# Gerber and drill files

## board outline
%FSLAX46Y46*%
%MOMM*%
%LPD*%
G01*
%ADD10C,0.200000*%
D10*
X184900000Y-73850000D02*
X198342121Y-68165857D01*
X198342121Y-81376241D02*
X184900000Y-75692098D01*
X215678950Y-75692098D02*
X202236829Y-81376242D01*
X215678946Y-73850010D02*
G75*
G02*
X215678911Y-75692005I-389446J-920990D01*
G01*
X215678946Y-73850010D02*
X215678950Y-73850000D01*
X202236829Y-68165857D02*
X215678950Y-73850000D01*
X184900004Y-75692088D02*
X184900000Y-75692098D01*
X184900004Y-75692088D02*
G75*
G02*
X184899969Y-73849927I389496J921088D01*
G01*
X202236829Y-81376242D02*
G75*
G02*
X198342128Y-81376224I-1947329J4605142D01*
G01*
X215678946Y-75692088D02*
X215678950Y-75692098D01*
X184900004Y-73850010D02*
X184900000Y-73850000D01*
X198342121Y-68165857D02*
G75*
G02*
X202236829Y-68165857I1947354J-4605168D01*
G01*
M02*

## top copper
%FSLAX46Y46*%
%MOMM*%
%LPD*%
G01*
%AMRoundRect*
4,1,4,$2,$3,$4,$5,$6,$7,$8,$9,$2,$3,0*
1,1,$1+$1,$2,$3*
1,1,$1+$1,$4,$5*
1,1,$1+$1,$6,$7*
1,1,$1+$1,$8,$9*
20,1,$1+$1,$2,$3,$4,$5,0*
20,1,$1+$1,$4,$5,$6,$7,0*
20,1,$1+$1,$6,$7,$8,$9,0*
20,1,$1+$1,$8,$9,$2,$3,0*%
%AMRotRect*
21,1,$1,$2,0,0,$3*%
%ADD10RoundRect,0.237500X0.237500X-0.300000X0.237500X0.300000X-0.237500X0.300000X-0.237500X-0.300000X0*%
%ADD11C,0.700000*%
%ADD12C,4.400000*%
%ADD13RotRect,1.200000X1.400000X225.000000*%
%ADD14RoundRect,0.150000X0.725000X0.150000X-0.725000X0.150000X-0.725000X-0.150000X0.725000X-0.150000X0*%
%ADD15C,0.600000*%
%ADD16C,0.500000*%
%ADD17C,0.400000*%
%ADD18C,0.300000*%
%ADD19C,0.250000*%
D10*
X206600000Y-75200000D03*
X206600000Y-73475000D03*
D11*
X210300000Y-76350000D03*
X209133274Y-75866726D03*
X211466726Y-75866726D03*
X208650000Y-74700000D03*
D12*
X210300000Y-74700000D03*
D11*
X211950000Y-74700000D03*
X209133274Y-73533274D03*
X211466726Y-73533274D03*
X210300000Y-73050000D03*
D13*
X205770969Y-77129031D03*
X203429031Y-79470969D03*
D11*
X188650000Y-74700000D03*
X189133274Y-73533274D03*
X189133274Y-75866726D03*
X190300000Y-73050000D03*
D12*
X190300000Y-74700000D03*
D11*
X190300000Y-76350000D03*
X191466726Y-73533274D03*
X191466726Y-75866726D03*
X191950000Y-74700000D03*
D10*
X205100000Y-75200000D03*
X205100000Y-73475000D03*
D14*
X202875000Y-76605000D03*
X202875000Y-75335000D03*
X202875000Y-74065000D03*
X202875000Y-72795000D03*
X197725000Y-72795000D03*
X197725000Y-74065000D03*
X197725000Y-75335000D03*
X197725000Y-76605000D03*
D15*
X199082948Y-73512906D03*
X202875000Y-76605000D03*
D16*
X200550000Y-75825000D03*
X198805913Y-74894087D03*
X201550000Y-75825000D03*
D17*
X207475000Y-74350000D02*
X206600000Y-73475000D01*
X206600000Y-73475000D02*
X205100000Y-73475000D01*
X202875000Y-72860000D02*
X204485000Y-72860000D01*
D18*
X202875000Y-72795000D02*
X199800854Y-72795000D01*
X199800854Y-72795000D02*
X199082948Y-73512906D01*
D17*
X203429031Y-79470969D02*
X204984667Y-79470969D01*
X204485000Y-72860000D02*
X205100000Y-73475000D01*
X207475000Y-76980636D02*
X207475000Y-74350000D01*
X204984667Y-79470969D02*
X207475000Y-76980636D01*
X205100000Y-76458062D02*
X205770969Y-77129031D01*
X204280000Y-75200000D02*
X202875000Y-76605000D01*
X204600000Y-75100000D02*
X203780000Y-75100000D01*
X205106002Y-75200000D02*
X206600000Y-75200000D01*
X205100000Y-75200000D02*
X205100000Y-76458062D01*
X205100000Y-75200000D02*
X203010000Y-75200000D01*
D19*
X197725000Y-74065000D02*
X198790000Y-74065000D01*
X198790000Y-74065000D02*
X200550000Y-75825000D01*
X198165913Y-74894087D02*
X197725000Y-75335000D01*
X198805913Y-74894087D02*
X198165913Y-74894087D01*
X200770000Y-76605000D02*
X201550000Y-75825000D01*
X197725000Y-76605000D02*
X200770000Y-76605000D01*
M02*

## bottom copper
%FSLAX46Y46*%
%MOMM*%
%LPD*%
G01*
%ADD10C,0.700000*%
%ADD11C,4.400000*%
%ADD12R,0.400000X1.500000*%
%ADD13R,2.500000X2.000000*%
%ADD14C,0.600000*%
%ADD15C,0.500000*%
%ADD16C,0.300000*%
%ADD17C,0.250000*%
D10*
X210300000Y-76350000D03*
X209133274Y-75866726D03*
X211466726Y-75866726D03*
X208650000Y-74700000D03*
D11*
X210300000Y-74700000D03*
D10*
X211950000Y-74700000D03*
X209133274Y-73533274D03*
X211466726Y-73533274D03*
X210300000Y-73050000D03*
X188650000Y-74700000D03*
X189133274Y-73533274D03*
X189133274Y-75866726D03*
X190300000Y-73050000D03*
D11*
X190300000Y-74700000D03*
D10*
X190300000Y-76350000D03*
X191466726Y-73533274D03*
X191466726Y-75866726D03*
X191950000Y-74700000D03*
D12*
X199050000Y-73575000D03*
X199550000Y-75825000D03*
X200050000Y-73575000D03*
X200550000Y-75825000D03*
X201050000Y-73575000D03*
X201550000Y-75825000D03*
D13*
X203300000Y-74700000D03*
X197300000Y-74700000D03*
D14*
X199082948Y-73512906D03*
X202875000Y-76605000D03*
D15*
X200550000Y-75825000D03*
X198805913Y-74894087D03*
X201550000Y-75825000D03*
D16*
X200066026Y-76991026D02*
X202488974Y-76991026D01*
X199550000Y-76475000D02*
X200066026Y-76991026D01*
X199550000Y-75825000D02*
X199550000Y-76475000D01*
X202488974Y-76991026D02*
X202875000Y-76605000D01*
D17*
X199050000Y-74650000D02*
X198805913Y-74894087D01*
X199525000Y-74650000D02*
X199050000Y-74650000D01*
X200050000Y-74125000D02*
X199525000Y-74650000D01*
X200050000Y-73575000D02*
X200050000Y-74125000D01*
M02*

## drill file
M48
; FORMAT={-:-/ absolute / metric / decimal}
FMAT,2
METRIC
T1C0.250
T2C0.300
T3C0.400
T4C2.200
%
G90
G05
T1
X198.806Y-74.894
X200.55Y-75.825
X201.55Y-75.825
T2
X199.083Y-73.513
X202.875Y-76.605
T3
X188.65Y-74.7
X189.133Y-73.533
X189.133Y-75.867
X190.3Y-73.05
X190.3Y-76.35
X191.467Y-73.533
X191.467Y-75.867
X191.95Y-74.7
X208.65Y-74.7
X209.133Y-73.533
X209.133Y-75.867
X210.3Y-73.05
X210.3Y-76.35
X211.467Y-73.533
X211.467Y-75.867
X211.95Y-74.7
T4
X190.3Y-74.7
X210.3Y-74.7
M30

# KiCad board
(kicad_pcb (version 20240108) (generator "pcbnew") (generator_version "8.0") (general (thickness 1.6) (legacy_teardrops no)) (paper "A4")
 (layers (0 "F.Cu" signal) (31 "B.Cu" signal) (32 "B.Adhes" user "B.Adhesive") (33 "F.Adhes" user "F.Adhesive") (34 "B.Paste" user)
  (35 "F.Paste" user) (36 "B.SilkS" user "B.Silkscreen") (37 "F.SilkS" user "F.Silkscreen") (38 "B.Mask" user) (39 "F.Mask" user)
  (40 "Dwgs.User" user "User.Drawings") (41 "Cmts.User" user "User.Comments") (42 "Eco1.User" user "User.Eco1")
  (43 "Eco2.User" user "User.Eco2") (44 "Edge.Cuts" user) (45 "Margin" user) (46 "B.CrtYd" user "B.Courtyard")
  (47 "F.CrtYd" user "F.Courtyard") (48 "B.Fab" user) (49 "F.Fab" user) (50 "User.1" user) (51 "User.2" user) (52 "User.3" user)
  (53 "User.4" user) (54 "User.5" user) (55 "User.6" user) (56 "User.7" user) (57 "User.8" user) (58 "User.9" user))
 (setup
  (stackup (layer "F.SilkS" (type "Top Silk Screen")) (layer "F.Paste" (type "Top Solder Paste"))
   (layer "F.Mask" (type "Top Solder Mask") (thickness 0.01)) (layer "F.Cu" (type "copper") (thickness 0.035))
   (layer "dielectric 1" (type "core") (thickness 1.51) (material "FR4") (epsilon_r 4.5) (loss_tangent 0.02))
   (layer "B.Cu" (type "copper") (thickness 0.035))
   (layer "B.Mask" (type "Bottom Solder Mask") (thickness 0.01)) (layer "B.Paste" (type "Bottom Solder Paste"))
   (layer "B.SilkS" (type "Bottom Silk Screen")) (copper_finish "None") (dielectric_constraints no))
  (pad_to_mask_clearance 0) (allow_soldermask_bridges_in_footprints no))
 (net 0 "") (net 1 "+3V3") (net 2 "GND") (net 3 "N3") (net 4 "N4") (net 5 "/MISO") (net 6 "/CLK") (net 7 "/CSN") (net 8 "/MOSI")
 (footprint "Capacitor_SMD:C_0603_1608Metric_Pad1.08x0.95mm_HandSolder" (layer "F.Cu") (at 206.6 74.3375 90)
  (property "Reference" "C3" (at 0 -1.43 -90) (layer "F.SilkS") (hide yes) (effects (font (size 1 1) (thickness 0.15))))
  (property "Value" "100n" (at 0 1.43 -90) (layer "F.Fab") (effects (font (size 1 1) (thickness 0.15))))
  (pad "1" smd roundrect (at -0.8625 0 90) (size 1.075 0.95) (layers "F.Cu" "F.Paste" "F.Mask") (roundrect_rratio 0.25) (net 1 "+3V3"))
  (pad "2" smd roundrect (at 0.8625 0 90) (size 1.075 0.95) (layers "F.Cu" "F.Paste" "F.Mask") (roundrect_rratio 0.25) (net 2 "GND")))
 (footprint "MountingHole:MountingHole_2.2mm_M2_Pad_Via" (layer "F.Cu") (at 210.3 74.7 90)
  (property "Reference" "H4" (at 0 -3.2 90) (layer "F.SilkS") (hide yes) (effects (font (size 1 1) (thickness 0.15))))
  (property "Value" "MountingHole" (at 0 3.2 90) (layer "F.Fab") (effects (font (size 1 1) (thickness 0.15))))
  (pad "1" thru_hole circle (at -1.65 0 90) (size 0.7 0.7) (drill 0.4) (layers "*.Cu" "*.Mask") (remove_unused_layers no) (zone_connect 2))
  (pad "1" thru_hole circle (at -1.166726 -1.166726 90) (size 0.7 0.7) (drill 0.4) (layers "*.Cu" "*.Mask") (remove_unused_layers no)
   (zone_connect 2))
  (pad "1" thru_hole circle (at -1.166726 1.166726 90) (size 0.7 0.7) (drill 0.4) (layers "*.Cu" "*.Mask") (remove_unused_layers no)
   (zone_connect 2))
  (pad "1" thru_hole circle (at 0 -1.65 90) (size 0.7 0.7) (drill 0.4) (layers "*.Cu" "*.Mask") (remove_unused_layers no) (zone_connect 2))
  (pad "1" thru_hole circle (at 0 0 90) (size 4.4 4.4) (drill 2.2) (layers "*.Cu" "*.Mask") (remove_unused_layers no))
  (pad "1" thru_hole circle (at 0 1.65 90) (size 0.7 0.7) (drill 0.4) (layers "*.Cu" "*.Mask") (remove_unused_layers no) (zone_connect 2))
  (pad "1" thru_hole circle (at 1.166726 -1.166726 90) (size 0.7 0.7) (drill 0.4) (layers "*.Cu" "*.Mask") (remove_unused_layers no)
   (zone_connect 2))
  (pad "1" thru_hole circle (at 1.166726 1.166726 90) (size 0.7 0.7) (drill 0.4) (layers "*.Cu" "*.Mask") (remove_unused_layers no)
   (zone_connect 2))
  (pad "1" thru_hole circle (at 1.65 0 90) (size 0.7 0.7) (drill 0.4) (layers "*.Cu" "*.Mask") (remove_unused_layers no) (zone_connect 2)))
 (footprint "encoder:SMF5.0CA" (layer "F.Cu") (at 204.6 78.3 -135)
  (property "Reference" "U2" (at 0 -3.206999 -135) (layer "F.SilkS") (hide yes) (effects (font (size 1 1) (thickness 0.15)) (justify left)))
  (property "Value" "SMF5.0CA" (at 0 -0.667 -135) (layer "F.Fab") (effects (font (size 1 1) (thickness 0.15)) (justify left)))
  (pad "1" smd rect (at -1.656 0 225) (size 1.2 1.4) (layers "F.Cu" "F.Paste" "F.Mask") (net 1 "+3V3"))
  (pad "2" smd rect (at 1.656 0 225) (size 1.2 1.4) (layers "F.Cu" "F.Paste" "F.Mask") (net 2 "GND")))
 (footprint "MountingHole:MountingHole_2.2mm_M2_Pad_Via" (layer "F.Cu") (at 190.3 74.7)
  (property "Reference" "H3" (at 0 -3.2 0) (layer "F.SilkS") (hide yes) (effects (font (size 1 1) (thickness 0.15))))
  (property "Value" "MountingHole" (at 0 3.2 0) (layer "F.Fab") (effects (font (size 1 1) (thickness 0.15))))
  (pad "1" thru_hole circle (at -1.65 0) (size 0.7 0.7) (drill 0.4) (layers "*.Cu" "*.Mask") (remove_unused_layers no) (zone_connect 2))
  (pad "1" thru_hole circle (at -1.166726 -1.166726) (size 0.7 0.7) (drill 0.4) (layers "*.Cu" "*.Mask") (remove_unused_layers no)
   (zone_connect 2))
  (pad "1" thru_hole circle (at -1.166726 1.166726) (size 0.7 0.7) (drill 0.4) (layers "*.Cu" "*.Mask") (remove_unused_layers no)
   (zone_connect 2))
  (pad "1" thru_hole circle (at 0 -1.65) (size 0.7 0.7) (drill 0.4) (layers "*.Cu" "*.Mask") (remove_unused_layers no) (zone_connect 2))
  (pad "1" thru_hole circle (at 0 0) (size 4.4 4.4) (drill 2.2) (layers "*.Cu" "*.Mask") (remove_unused_layers no))
  (pad "1" thru_hole circle (at 0 1.65) (size 0.7 0.7) (drill 0.4) (layers "*.Cu" "*.Mask") (remove_unused_layers no) (zone_connect 2))
  (pad "1" thru_hole circle (at 1.166726 -1.166726) (size 0.7 0.7) (drill 0.4) (layers "*.Cu" "*.Mask") (remove_unused_layers no)
   (zone_connect 2))
  (pad "1" thru_hole circle (at 1.166726 1.166726) (size 0.7 0.7) (drill 0.4) (layers "*.Cu" "*.Mask") (remove_unused_layers no)
   (zone_connect 2))
  (pad "1" thru_hole circle (at 1.65 0) (size 0.7 0.7) (drill 0.4) (layers "*.Cu" "*.Mask") (remove_unused_layers no) (zone_connect 2)))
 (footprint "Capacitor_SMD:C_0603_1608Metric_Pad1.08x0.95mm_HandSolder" (layer "F.Cu") (at 205.1 74.3375 90)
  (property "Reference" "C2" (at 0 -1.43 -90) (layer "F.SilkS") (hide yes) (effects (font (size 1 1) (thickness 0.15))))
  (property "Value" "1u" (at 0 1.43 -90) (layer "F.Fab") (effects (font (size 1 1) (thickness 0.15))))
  (pad "1" smd roundrect (at -0.8625 0 90) (size 1.075 0.95) (layers "F.Cu" "F.Paste" "F.Mask") (roundrect_rratio 0.25) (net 1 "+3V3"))
  (pad "2" smd roundrect (at 0.8625 0 90) (size 1.075 0.95) (layers "F.Cu" "F.Paste" "F.Mask") (roundrect_rratio 0.25) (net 2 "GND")))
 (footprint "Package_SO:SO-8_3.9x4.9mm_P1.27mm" (layer "F.Cu") (at 200.3 74.7 180)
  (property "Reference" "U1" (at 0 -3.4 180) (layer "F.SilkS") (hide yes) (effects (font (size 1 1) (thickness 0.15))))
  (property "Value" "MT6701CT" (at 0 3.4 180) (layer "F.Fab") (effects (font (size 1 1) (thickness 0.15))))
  (pad "1" smd roundrect (at -2.575 -1.905 180) (size 1.75 0.6) (layers "F.Cu" "F.Paste" "F.Mask") (roundrect_rratio 0.25) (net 1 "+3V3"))
  (pad "2" smd roundrect (at -2.575 -0.635 180) (size 1.75 0.6) (layers "F.Cu" "F.Paste" "F.Mask") (roundrect_rratio 0.25) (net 1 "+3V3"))
  (pad "3" smd roundrect (at -2.575 0.635 180) (size 1.75 0.6) (layers "F.Cu" "F.Paste" "F.Mask") (roundrect_rratio 0.25) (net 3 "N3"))
  (pad "4" smd roundrect (at -2.575 1.905 180) (size 1.75 0.6) (layers "F.Cu" "F.Paste" "F.Mask") (roundrect_rratio 0.25) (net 2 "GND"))
  (pad "5" smd roundrect (at 2.575 1.905 180) (size 1.75 0.6) (layers "F.Cu" "F.Paste" "F.Mask") (roundrect_rratio 0.25) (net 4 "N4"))
  (pad "6" smd roundrect (at 2.575 0.635 180) (size 1.75 0.6) (layers "F.Cu" "F.Paste" "F.Mask") (roundrect_rratio 0.25) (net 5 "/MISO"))
  (pad "7" smd roundrect (at 2.575 -0.635 180) (size 1.75 0.6) (layers "F.Cu" "F.Paste" "F.Mask") (roundrect_rratio 0.25) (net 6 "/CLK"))
  (pad "8" smd roundrect (at 2.575 -1.905 180) (size 1.75 0.6) (layers "F.Cu" "F.Paste" "F.Mask") (roundrect_rratio 0.25) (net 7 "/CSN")))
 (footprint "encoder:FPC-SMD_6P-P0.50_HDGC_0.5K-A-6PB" (layer "B.Cu") (at 200.3 74.7)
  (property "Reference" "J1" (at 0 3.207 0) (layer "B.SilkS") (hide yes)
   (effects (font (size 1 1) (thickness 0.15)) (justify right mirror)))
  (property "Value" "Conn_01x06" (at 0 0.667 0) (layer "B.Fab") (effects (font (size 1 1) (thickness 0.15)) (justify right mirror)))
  (pad "1" smd rect (at -1.25 -1.125 180) (size 0.4 1.5) (layers "B.Cu" "B.Paste" "B.Mask") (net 2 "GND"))
  (pad "2" smd rect (at -0.75 1.125 180) (size 0.4 1.5) (layers "B.Cu" "B.Paste" "B.Mask") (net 1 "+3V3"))
  (pad "3" smd rect (at -0.25 -1.125 180) (size 0.4 1.5) (layers "B.Cu" "B.Paste" "B.Mask") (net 6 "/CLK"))
  (pad "4" smd rect (at 0.25 1.125 180) (size 0.4 1.5) (layers "B.Cu" "B.Paste" "B.Mask") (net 5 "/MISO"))
  (pad "5" smd rect (at 0.75 -1.125 180) (size 0.4 1.5) (layers "B.Cu" "B.Paste" "B.Mask") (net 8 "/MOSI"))
  (pad "6" smd rect (at 1.25 1.125 180) (size 0.4 1.5) (layers "B.Cu" "B.Paste" "B.Mask") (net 7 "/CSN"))
  (pad "7" smd rect (at 3 0 180) (size 2.5 2) (layers "B.Cu" "B.Paste" "B.Mask"))
  (pad "8" smd rect (at -3 0) (size 2.5 2) (layers "B.Cu" "B.Paste" "B.Mask")))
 (gr_line (start 184.9 73.85) (end 198.342121 68.165857) (stroke (width 0.2) (type default)) (layer "Edge.Cuts"))
 (gr_line (start 198.342121 81.376241) (end 184.9 75.692098) (stroke (width 0.2) (type default)) (layer "Edge.Cuts"))
 (gr_line (start 215.67895 75.692098) (end 202.236829 81.376242) (stroke (width 0.2) (type default)) (layer "Edge.Cuts"))
 (gr_arc (start 215.678946 73.85001) (mid 216.289475 74.771049) (end 215.678946 75.692088) (stroke (width 0.2) (type default))
  (layer "Edge.Cuts"))
 (gr_line (start 215.678946 73.85001) (end 215.67895 73.85) (stroke (width 0.2) (type default)) (layer "Edge.Cuts"))
 (gr_line (start 202.236829 68.165857) (end 215.67895 73.85) (stroke (width 0.2) (type default)) (layer "Edge.Cuts"))
 (gr_line (start 184.900004 75.692088) (end 184.9 75.692098) (stroke (width 0.2) (type default)) (layer "Edge.Cuts"))
 (gr_arc (start 184.900004 75.692088) (mid 184.289475 74.771049) (end 184.900004 73.85001) (stroke (width 0.2) (type default))
  (layer "Edge.Cuts"))
 (gr_arc (start 202.236829 81.376242) (mid 200.289475 81.771049) (end 198.342121 81.376241) (stroke (width 0.2) (type default))
  (layer "Edge.Cuts"))
 (gr_line (start 215.678946 75.692088) (end 215.67895 75.692098) (stroke (width 0.2) (type default)) (layer "Edge.Cuts"))
 (gr_line (start 184.900004 73.85001) (end 184.9 73.85) (stroke (width 0.2) (type default)) (layer "Edge.Cuts"))
 (gr_arc (start 198.342121 68.165857) (mid 200.289475 67.771049) (end 202.236829 68.165857) (stroke (width 0.2) (type default))
  (layer "Edge.Cuts"))
 (segment (start 207.475 74.35) (end 206.6 73.475) (width 0.4) (layer "F.Cu") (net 2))
 (segment (start 206.6 73.475) (end 205.1 73.475) (width 0.4) (layer "F.Cu") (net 2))
 (segment (start 202.875 72.86) (end 204.485 72.86) (width 0.4) (layer "F.Cu") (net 2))
 (segment (start 202.875 72.795) (end 199.800854 72.795) (width 0.3) (layer "F.Cu") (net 2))
 (segment (start 199.800854 72.795) (end 199.082948 73.512906) (width 0.3) (layer "F.Cu") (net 2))
 (segment (start 203.429031 79.470969) (end 204.984667 79.470969) (width 0.4) (layer "F.Cu") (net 2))
 (segment (start 204.485 72.86) (end 205.1 73.475) (width 0.4) (layer "F.Cu") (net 2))
 (segment (start 207.475 76.980636) (end 207.475 74.35) (width 0.4) (layer "F.Cu") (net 2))
 (segment (start 204.984667 79.470969) (end 207.475 76.980636) (width 0.4) (layer "F.Cu") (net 2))
 (via (at 199.082948 73.512906) (size 0.6) (drill 0.3) (layers "F.Cu" "B.Cu") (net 2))
 (segment (start 205.1 76.458062) (end 205.770969 77.129031) (width 0.4) (layer "F.Cu") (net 1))
 (segment (start 204.28 75.2) (end 202.875 76.605) (width 0.4) (layer "F.Cu") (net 1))
 (segment (start 204.6 75.1) (end 203.78 75.1) (width 0.4) (layer "F.Cu") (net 1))
 (segment (start 205.106002 75.2) (end 206.6 75.2) (width 0.4) (layer "F.Cu") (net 1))
 (segment (start 205.1 75.2) (end 205.1 76.458062) (width 0.4) (layer "F.Cu") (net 1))
 (segment (start 205.1 75.2) (end 203.01 75.2) (width 0.4) (layer "F.Cu") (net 1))
 (via (at 202.875 76.605) (size 0.6) (drill 0.3) (layers "F.Cu" "B.Cu") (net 1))
 (segment (start 200.066026 76.991026) (end 202.488974 76.991026) (width 0.3) (layer "B.Cu") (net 1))
 (segment (start 199.55 76.475) (end 200.066026 76.991026) (width 0.3) (layer "B.Cu") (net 1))
 (segment (start 199.55 75.825) (end 199.55 76.475) (width 0.3) (layer "B.Cu") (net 1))
 (segment (start 202.488974 76.991026) (end 202.875 76.605) (width 0.3) (layer "B.Cu") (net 1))
 (segment (start 197.725 74.065) (end 198.79 74.065) (width 0.25) (layer "F.Cu") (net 5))
 (segment (start 198.79 74.065) (end 200.55 75.825) (width 0.25) (layer "F.Cu") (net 5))
 (via (at 200.55 75.825) (size 0.5) (drill 0.25) (layers "F.Cu" "B.Cu") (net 5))
 (segment (start 198.165913 74.894087) (end 197.725 75.335) (width 0.25) (layer "F.Cu") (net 6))
 (segment (start 198.805913 74.894087) (end 198.165913 74.894087) (width 0.25) (layer "F.Cu") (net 6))
 (via (at 198.805913 74.894087) (size 0.5) (drill 0.25) (layers "F.Cu" "B.Cu") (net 6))
 (segment (start 199.05 74.65) (end 198.805913 74.894087) (width 0.25) (layer "B.Cu") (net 6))
 (segment (start 199.525 74.65) (end 199.05 74.65) (width 0.25) (layer "B.Cu") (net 6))
 (segment (start 200.05 74.125) (end 199.525 74.65) (width 0.25) (layer "B.Cu") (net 6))
 (segment (start 200.05 73.575) (end 200.05 74.125) (width 0.25) (layer "B.Cu") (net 6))
 (segment (start 200.77 76.605) (end 201.55 75.825) (width 0.25) (layer "F.Cu") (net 7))
 (segment (start 197.725 76.605) (end 200.77 76.605) (width 0.25) (layer "F.Cu") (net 7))
 (via (at 201.55 75.825) (size 0.5) (drill 0.25) (layers "F.Cu" "B.Cu") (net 7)))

